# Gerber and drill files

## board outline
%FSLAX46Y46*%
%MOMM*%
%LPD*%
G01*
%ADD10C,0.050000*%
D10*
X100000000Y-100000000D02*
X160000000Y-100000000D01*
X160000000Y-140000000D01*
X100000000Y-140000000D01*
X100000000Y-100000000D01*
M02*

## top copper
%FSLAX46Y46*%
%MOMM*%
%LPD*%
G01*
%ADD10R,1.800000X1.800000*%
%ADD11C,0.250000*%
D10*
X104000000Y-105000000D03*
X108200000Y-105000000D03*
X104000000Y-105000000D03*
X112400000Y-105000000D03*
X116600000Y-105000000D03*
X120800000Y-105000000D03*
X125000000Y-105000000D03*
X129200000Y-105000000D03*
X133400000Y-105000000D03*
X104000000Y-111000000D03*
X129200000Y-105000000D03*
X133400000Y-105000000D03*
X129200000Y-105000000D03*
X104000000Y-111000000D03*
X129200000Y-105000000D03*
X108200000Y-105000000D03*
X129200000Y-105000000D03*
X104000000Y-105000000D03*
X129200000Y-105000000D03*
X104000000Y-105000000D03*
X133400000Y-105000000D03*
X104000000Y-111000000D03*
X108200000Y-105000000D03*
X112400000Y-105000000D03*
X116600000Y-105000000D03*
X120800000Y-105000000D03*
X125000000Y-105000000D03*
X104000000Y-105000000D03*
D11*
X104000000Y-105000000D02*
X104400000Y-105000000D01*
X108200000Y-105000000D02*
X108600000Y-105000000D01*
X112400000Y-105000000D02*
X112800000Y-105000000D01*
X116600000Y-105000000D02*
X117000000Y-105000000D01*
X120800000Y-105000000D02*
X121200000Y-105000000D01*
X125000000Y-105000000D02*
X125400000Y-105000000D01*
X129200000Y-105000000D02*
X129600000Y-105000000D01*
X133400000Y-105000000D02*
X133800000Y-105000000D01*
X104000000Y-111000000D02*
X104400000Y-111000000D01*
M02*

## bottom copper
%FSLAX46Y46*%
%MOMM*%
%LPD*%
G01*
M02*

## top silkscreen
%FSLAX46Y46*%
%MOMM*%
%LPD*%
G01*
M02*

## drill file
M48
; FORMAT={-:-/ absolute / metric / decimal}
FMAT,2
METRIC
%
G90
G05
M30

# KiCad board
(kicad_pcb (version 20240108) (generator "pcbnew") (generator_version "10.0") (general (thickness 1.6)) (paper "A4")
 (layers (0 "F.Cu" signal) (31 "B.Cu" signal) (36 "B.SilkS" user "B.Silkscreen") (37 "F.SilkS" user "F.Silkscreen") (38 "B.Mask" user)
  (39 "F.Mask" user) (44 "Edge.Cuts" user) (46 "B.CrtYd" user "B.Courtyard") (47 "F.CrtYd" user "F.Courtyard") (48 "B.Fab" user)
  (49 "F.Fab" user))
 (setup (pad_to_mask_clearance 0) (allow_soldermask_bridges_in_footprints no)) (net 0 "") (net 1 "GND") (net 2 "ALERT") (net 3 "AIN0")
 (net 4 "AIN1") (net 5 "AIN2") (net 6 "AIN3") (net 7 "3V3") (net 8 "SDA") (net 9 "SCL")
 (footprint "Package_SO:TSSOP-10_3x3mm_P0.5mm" (layer "F.Cu") (at 100 100)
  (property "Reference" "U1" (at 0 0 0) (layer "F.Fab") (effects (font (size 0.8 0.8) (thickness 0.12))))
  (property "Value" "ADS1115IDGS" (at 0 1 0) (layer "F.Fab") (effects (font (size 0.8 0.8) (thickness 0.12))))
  (pad "1" smd rect (at 4.000 5.000) (size 1.8 1.8) (layers "F.Cu" "F.Paste" "F.Mask") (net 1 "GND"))
  (pad "2" smd rect (at 8.200 5.000) (size 1.8 1.8) (layers "F.Cu" "F.Paste" "F.Mask") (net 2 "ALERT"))
  (pad "3" smd rect (at 4.000 5.000) (size 1.8 1.8) (layers "F.Cu" "F.Paste" "F.Mask") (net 1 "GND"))
  (pad "4" smd rect (at 12.400 5.000) (size 1.8 1.8) (layers "F.Cu" "F.Paste" "F.Mask") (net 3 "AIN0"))
  (pad "5" smd rect (at 16.600 5.000) (size 1.8 1.8) (layers "F.Cu" "F.Paste" "F.Mask") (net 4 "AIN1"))
  (pad "6" smd rect (at 20.800 5.000) (size 1.8 1.8) (layers "F.Cu" "F.Paste" "F.Mask") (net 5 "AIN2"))
  (pad "7" smd rect (at 25.000 5.000) (size 1.8 1.8) (layers "F.Cu" "F.Paste" "F.Mask") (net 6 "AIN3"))
  (pad "8" smd rect (at 29.200 5.000) (size 1.8 1.8) (layers "F.Cu" "F.Paste" "F.Mask") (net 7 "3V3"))
  (pad "9" smd rect (at 33.400 5.000) (size 1.8 1.8) (layers "F.Cu" "F.Paste" "F.Mask") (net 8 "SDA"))
  (pad "10" smd rect (at 4.000 11.000) (size 1.8 1.8) (layers "F.Cu" "F.Paste" "F.Mask") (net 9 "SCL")))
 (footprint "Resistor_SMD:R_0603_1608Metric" (layer "F.Cu") (at 100 100)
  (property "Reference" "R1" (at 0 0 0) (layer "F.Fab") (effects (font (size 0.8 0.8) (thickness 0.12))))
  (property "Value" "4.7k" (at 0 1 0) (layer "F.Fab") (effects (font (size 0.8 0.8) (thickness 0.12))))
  (pad "1" smd rect (at 29.200 5.000) (size 1.8 1.8) (layers "F.Cu" "F.Paste" "F.Mask") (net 7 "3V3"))
  (pad "2" smd rect (at 33.400 5.000) (size 1.8 1.8) (layers "F.Cu" "F.Paste" "F.Mask") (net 8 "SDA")))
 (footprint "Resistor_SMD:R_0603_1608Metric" (layer "F.Cu") (at 100 100)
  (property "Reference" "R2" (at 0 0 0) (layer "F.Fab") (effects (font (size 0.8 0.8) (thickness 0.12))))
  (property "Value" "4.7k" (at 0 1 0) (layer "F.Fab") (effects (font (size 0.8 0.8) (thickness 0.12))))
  (pad "1" smd rect (at 29.200 5.000) (size 1.8 1.8) (layers "F.Cu" "F.Paste" "F.Mask") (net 7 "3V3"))
  (pad "2" smd rect (at 4.000 11.000) (size 1.8 1.8) (layers "F.Cu" "F.Paste" "F.Mask") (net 9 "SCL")))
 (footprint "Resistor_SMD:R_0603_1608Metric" (layer "F.Cu") (at 100 100)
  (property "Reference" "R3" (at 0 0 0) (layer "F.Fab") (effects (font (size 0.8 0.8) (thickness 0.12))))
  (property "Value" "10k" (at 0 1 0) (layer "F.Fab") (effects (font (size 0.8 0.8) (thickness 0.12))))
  (pad "1" smd rect (at 29.200 5.000) (size 1.8 1.8) (layers "F.Cu" "F.Paste" "F.Mask") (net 7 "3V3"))
  (pad "2" smd rect (at 8.200 5.000) (size 1.8 1.8) (layers "F.Cu" "F.Paste" "F.Mask") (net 2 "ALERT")))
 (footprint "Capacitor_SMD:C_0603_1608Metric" (layer "F.Cu") (at 100 100)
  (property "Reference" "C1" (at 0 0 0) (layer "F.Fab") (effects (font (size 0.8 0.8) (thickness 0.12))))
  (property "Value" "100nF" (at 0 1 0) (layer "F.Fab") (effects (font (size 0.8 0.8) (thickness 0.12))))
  (pad "1" smd rect (at 29.200 5.000) (size 1.8 1.8) (layers "F.Cu" "F.Paste" "F.Mask") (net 7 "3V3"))
  (pad "2" smd rect (at 4.000 5.000) (size 1.8 1.8) (layers "F.Cu" "F.Paste" "F.Mask") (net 1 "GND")))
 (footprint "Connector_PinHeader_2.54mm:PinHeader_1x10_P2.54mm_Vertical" (layer "F.Cu") (at 100 100)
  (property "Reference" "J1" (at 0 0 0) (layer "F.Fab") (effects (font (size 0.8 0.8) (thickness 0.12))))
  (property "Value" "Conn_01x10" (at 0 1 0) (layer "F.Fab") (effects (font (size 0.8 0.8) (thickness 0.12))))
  (pad "1" smd rect (at 29.200 5.000) (size 1.8 1.8) (layers "F.Cu" "F.Paste" "F.Mask") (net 7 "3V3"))
  (pad "2" smd rect (at 4.000 5.000) (size 1.8 1.8) (layers "F.Cu" "F.Paste" "F.Mask") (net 1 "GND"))
  (pad "3" smd rect (at 33.400 5.000) (size 1.8 1.8) (layers "F.Cu" "F.Paste" "F.Mask") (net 8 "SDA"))
  (pad "4" smd rect (at 4.000 11.000) (size 1.8 1.8) (layers "F.Cu" "F.Paste" "F.Mask") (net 9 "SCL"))
  (pad "5" smd rect (at 8.200 5.000) (size 1.8 1.8) (layers "F.Cu" "F.Paste" "F.Mask") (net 2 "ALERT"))
  (pad "6" smd rect (at 12.400 5.000) (size 1.8 1.8) (layers "F.Cu" "F.Paste" "F.Mask") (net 3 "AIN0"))
  (pad "7" smd rect (at 16.600 5.000) (size 1.8 1.8) (layers "F.Cu" "F.Paste" "F.Mask") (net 4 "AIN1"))
  (pad "8" smd rect (at 20.800 5.000) (size 1.8 1.8) (layers "F.Cu" "F.Paste" "F.Mask") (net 5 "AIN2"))
  (pad "9" smd rect (at 25.000 5.000) (size 1.8 1.8) (layers "F.Cu" "F.Paste" "F.Mask") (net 6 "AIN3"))
  (pad "10" smd rect (at 4.000 5.000) (size 1.8 1.8) (layers "F.Cu" "F.Paste" "F.Mask") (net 1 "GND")))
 (gr_rect (start 100 100) (end 160 140) (stroke (width 0.05) (type default)) (fill none) (layer "Edge.Cuts"))
 (segment (start 104.000 105.000) (end 104.400 105.000) (width 0.25) (layer "F.Cu") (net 1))
 (segment (start 108.200 105.000) (end 108.600 105.000) (width 0.25) (layer "F.Cu") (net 2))
 (segment (start 112.400 105.000) (end 112.800 105.000) (width 0.25) (layer "F.Cu") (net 3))
 (segment (start 116.600 105.000) (end 117.000 105.000) (width 0.25) (layer "F.Cu") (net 4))
 (segment (start 120.800 105.000) (end 121.200 105.000) (width 0.25) (layer "F.Cu") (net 5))
 (segment (start 125.000 105.000) (end 125.400 105.000) (width 0.25) (layer "F.Cu") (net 6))
 (segment (start 129.200 105.000) (end 129.600 105.000) (width 0.25) (layer "F.Cu") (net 7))
 (segment (start 133.400 105.000) (end 133.800 105.000) (width 0.25) (layer "F.Cu") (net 8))
 (segment (start 104.000 111.000) (end 104.400 111.000) (width 0.25) (layer "F.Cu") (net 9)))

